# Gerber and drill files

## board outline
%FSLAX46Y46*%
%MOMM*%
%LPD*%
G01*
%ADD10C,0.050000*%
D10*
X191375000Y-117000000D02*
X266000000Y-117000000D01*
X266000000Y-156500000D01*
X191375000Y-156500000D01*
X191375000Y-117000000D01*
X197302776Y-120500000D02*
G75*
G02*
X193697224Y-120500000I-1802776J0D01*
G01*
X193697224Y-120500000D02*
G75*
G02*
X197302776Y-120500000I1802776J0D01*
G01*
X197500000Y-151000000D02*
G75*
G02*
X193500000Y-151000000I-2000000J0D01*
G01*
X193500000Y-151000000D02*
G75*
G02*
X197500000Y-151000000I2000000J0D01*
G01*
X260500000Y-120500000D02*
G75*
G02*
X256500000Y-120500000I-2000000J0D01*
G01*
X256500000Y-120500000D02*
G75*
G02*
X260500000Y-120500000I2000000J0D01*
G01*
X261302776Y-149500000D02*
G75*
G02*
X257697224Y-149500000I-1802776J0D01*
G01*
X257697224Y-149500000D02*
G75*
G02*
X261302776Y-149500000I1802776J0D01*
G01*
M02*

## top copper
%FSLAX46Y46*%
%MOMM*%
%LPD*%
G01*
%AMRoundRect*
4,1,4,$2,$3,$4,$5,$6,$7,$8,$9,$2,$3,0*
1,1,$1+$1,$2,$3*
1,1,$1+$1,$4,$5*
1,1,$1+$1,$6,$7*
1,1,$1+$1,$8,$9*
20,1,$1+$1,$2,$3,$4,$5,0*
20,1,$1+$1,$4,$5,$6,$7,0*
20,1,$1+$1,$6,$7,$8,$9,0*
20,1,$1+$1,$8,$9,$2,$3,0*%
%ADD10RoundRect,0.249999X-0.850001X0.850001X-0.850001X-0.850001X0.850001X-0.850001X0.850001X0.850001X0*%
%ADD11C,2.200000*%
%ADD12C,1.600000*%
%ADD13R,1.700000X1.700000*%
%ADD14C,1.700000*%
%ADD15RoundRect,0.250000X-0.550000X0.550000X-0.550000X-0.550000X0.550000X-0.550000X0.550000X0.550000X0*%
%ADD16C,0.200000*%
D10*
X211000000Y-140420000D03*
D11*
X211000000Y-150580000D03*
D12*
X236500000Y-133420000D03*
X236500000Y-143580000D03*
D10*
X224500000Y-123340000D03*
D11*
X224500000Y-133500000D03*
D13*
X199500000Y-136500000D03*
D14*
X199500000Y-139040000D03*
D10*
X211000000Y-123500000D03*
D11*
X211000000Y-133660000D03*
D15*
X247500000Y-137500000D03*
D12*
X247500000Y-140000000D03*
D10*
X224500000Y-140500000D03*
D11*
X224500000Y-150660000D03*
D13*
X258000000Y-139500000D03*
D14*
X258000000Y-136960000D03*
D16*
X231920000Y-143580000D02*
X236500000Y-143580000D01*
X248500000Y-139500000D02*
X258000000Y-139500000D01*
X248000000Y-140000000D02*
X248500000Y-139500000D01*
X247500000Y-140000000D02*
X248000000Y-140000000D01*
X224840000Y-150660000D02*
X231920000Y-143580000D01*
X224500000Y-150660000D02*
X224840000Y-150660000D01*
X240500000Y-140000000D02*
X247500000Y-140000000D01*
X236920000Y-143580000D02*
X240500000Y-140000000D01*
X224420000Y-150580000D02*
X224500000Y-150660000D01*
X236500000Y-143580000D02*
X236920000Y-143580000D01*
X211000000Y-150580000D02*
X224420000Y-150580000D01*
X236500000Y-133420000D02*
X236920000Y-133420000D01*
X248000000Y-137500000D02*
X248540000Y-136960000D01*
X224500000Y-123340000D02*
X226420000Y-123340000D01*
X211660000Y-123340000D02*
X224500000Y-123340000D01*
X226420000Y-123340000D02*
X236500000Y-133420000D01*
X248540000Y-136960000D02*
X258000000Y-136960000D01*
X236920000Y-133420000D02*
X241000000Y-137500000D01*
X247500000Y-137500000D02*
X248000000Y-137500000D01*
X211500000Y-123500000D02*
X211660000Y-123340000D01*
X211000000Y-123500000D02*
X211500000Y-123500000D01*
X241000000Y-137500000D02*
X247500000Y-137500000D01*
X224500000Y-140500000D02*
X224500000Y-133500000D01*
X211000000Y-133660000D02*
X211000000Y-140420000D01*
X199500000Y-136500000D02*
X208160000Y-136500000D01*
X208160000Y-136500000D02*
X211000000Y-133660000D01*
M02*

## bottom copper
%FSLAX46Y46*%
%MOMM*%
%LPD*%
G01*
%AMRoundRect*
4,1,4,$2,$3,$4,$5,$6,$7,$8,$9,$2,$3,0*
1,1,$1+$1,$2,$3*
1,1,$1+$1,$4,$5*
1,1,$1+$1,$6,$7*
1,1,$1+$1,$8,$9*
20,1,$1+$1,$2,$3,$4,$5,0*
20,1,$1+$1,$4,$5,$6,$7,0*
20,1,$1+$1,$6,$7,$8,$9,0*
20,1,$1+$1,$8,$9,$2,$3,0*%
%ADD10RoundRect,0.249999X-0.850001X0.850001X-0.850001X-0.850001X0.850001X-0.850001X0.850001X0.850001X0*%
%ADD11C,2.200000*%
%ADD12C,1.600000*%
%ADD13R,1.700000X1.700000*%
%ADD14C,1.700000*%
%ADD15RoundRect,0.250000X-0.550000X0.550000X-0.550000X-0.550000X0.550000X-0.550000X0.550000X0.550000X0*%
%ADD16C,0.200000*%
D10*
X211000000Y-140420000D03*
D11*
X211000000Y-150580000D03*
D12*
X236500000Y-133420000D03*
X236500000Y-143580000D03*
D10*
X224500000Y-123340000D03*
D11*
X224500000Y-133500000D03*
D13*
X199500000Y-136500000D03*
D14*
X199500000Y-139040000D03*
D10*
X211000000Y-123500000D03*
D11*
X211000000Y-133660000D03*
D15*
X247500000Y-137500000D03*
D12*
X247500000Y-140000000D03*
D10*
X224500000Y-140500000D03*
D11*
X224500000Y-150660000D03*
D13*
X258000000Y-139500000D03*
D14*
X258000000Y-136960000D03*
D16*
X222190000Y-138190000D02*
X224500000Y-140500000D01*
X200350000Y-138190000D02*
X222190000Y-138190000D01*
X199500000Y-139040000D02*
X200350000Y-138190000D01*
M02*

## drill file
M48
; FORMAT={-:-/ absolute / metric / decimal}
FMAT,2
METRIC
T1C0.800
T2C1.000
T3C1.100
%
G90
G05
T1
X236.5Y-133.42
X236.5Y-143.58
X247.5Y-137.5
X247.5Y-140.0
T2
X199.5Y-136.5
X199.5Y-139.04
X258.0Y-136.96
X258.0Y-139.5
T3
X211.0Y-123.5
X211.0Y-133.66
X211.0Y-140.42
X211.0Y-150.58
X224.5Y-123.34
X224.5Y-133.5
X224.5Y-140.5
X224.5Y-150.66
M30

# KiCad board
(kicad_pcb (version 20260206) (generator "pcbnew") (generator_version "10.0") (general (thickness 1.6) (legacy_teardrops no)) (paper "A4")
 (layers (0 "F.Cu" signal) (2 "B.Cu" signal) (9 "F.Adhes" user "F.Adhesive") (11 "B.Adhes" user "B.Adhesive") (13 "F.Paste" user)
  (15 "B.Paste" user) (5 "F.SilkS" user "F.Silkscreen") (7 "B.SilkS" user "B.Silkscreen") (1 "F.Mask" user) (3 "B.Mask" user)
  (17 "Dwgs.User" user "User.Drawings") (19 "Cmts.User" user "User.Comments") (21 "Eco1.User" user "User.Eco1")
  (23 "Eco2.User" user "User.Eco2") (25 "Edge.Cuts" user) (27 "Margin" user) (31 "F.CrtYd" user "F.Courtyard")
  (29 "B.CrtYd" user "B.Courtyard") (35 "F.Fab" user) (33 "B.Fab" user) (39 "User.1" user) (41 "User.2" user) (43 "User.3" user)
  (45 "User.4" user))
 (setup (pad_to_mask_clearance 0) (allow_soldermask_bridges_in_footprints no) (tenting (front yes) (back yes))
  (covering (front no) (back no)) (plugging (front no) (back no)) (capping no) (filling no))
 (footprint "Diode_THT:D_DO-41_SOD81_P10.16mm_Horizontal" (layer "F.Cu") (at 211 140.42 -90)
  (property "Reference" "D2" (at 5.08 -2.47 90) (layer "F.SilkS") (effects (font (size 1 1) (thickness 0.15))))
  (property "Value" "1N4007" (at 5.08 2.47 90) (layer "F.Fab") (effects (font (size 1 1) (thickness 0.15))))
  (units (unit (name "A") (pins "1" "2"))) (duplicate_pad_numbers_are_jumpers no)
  (pad "1" thru_hole roundrect (at 0 0 270) (size 2.2 2.2) (drill 1.1) (layers "*.Cu" "*.Mask") (remove_unused_layers no)
   (roundrect_rratio 0.113636) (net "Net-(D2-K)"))
  (pad "2" thru_hole circle (at 10.16 0 270) (size 2.2 2.2) (drill 1.1) (layers "*.Cu" "*.Mask") (remove_unused_layers no) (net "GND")))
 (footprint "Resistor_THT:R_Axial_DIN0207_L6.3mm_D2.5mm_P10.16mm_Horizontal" (layer "F.Cu") (at 236.5 133.42 -90)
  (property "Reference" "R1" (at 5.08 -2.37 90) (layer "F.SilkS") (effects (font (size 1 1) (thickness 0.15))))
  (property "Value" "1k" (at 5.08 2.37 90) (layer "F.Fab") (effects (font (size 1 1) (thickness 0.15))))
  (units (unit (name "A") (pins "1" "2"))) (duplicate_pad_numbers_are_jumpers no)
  (pad "1" thru_hole circle (at 0 0 270) (size 1.6 1.6) (drill 0.8) (layers "*.Cu" "*.Mask") (remove_unused_layers no) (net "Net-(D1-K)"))
  (pad "2" thru_hole circle (at 10.16 0 270) (size 1.6 1.6) (drill 0.8) (layers "*.Cu" "*.Mask") (remove_unused_layers no) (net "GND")))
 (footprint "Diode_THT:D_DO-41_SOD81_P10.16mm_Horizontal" (layer "F.Cu") (at 224.5 123.34 -90)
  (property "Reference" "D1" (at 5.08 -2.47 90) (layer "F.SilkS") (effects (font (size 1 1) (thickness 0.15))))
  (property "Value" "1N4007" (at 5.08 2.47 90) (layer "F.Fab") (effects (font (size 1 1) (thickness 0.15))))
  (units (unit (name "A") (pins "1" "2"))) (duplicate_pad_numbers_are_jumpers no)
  (pad "1" thru_hole roundrect (at 0 0 270) (size 2.2 2.2) (drill 1.1) (layers "*.Cu" "*.Mask") (remove_unused_layers no)
   (roundrect_rratio 0.113636) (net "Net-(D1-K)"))
  (pad "2" thru_hole circle (at 10.16 0 270) (size 2.2 2.2) (drill 1.1) (layers "*.Cu" "*.Mask") (remove_unused_layers no)
   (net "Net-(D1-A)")))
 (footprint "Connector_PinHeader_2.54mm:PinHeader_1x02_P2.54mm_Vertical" (layer "F.Cu") (at 199.5 136.5)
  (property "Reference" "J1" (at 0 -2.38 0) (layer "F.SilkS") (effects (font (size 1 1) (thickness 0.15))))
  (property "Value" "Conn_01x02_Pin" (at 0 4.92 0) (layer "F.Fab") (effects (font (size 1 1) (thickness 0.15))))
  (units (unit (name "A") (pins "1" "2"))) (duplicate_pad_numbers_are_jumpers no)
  (pad "1" thru_hole rect (at 0 0) (size 1.7 1.7) (drill 1) (layers "*.Cu" "*.Mask") (remove_unused_layers no) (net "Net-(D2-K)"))
  (pad "2" thru_hole circle (at 0 2.54) (size 1.7 1.7) (drill 1) (layers "*.Cu" "*.Mask") (remove_unused_layers no) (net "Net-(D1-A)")))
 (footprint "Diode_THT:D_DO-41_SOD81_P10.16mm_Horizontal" (layer "F.Cu") (at 211 123.5 -90)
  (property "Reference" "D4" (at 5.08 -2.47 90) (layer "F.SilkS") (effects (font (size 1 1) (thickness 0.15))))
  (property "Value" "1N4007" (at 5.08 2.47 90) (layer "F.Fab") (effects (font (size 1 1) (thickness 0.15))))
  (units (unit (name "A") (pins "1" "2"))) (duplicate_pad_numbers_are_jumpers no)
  (pad "1" thru_hole roundrect (at 0 0 270) (size 2.2 2.2) (drill 1.1) (layers "*.Cu" "*.Mask") (remove_unused_layers no)
   (roundrect_rratio 0.113636) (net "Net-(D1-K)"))
  (pad "2" thru_hole circle (at 10.16 0 270) (size 2.2 2.2) (drill 1.1) (layers "*.Cu" "*.Mask") (remove_unused_layers no)
   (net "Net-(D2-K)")))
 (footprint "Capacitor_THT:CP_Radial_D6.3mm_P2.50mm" (layer "F.Cu") (at 247.5 137.5 -90)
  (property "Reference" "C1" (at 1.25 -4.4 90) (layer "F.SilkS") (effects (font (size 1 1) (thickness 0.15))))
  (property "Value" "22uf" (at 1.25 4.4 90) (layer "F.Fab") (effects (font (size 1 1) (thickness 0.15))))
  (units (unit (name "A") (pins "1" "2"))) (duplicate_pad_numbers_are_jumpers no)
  (pad "1" thru_hole roundrect (at 0 0 270) (size 1.6 1.6) (drill 0.8) (layers "*.Cu" "*.Mask") (remove_unused_layers no)
   (roundrect_rratio 0.15625) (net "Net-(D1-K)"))
  (pad "2" thru_hole circle (at 2.5 0 270) (size 1.6 1.6) (drill 0.8) (layers "*.Cu" "*.Mask") (remove_unused_layers no) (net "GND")))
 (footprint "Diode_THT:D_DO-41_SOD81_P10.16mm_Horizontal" (layer "F.Cu") (at 224.5 140.5 -90)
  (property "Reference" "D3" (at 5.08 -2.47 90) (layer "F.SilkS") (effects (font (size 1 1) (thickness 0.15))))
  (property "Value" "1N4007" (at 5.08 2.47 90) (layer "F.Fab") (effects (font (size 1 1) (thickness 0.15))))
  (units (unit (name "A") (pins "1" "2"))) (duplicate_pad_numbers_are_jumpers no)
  (pad "1" thru_hole roundrect (at 0 0 270) (size 2.2 2.2) (drill 1.1) (layers "*.Cu" "*.Mask") (remove_unused_layers no)
   (roundrect_rratio 0.113636) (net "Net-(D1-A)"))
  (pad "2" thru_hole circle (at 10.16 0 270) (size 2.2 2.2) (drill 1.1) (layers "*.Cu" "*.Mask") (remove_unused_layers no) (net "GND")))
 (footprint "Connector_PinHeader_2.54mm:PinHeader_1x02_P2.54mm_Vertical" (layer "F.Cu") (at 258 139.5 180)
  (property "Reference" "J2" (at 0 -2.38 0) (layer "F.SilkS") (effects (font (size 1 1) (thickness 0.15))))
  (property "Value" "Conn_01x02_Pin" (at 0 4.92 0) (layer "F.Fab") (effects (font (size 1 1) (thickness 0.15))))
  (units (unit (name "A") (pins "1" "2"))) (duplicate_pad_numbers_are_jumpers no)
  (pad "1" thru_hole rect (at 0 0 180) (size 1.7 1.7) (drill 1) (layers "*.Cu" "*.Mask") (remove_unused_layers no) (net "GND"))
  (pad "2" thru_hole circle (at 0 2.54 180) (size 1.7 1.7) (drill 1) (layers "*.Cu" "*.Mask") (remove_unused_layers no) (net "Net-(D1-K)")))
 (gr_rect (start 191.375 117) (end 266 156.5) (stroke (width 0.05) (type default)) (fill no) (layer "Edge.Cuts"))
 (gr_circle (center 195.5 120.5) (end 196.5 122) (stroke (width 0.05) (type default)) (fill no) (layer "Edge.Cuts"))
 (gr_circle (center 195.5 151) (end 195.5 153) (stroke (width 0.05) (type default)) (fill no) (layer "Edge.Cuts"))
 (gr_circle (center 258.5 120.5) (end 258.5 122.5) (stroke (width 0.05) (type default)) (fill no) (layer "Edge.Cuts"))
 (gr_circle (center 259.5 149.5) (end 258.5 151) (stroke (width 0.05) (type default)) (fill no) (layer "Edge.Cuts"))
 (segment (start 231.92 143.58) (end 236.5 143.58) (width 0.2) (layer "F.Cu") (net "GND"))
 (segment (start 248.5 139.5) (end 258 139.5) (width 0.2) (layer "F.Cu") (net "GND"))
 (segment (start 248 140) (end 248.5 139.5) (width 0.2) (layer "F.Cu") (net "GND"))
 (segment (start 247.5 140) (end 248 140) (width 0.2) (layer "F.Cu") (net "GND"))
 (segment (start 224.84 150.66) (end 231.92 143.58) (width 0.2) (layer "F.Cu") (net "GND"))
 (segment (start 224.5 150.66) (end 224.84 150.66) (width 0.2) (layer "F.Cu") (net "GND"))
 (segment (start 240.5 140) (end 247.5 140) (width 0.2) (layer "F.Cu") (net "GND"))
 (segment (start 236.92 143.58) (end 240.5 140) (width 0.2) (layer "F.Cu") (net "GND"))
 (segment (start 224.42 150.58) (end 224.5 150.66) (width 0.2) (layer "F.Cu") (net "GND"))
 (segment (start 236.5 143.58) (end 236.92 143.58) (width 0.2) (layer "F.Cu") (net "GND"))
 (segment (start 211 150.58) (end 224.42 150.58) (width 0.2) (layer "F.Cu") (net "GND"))
 (segment (start 236.5 133.42) (end 236.92 133.42) (width 0.2) (layer "F.Cu") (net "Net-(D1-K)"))
 (segment (start 248 137.5) (end 248.54 136.96) (width 0.2) (layer "F.Cu") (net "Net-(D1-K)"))
 (segment (start 224.5 123.34) (end 226.42 123.34) (width 0.2) (layer "F.Cu") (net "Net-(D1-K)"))
 (segment (start 211.66 123.34) (end 224.5 123.34) (width 0.2) (layer "F.Cu") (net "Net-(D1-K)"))
 (segment (start 226.42 123.34) (end 236.5 133.42) (width 0.2) (layer "F.Cu") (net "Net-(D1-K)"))
 (segment (start 248.54 136.96) (end 258 136.96) (width 0.2) (layer "F.Cu") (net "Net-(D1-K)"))
 (segment (start 236.92 133.42) (end 241 137.5) (width 0.2) (layer "F.Cu") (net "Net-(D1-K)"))
 (segment (start 247.5 137.5) (end 248 137.5) (width 0.2) (layer "F.Cu") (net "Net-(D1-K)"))
 (segment (start 211.5 123.5) (end 211.66 123.34) (width 0.2) (layer "F.Cu") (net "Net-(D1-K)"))
 (segment (start 211 123.5) (end 211.5 123.5) (width 0.2) (layer "F.Cu") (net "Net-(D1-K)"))
 (segment (start 241 137.5) (end 247.5 137.5) (width 0.2) (layer "F.Cu") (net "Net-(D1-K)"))
 (segment (start 224.5 140.5) (end 224.5 133.5) (width 0.2) (layer "F.Cu") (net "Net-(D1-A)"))
 (segment (start 222.19 138.19) (end 224.5 140.5) (width 0.2) (layer "B.Cu") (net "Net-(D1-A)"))
 (segment (start 200.35 138.19) (end 222.19 138.19) (width 0.2) (layer "B.Cu") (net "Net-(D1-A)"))
 (segment (start 199.5 139.04) (end 200.35 138.19) (width 0.2) (layer "B.Cu") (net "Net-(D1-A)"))
 (segment (start 211 133.66) (end 211 140.42) (width 0.2) (layer "F.Cu") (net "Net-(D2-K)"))
 (segment (start 199.5 136.5) (end 208.16 136.5) (width 0.2) (layer "F.Cu") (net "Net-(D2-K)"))
 (segment (start 208.16 136.5) (end 211 133.66) (width 0.2) (layer "F.Cu") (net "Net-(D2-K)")))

